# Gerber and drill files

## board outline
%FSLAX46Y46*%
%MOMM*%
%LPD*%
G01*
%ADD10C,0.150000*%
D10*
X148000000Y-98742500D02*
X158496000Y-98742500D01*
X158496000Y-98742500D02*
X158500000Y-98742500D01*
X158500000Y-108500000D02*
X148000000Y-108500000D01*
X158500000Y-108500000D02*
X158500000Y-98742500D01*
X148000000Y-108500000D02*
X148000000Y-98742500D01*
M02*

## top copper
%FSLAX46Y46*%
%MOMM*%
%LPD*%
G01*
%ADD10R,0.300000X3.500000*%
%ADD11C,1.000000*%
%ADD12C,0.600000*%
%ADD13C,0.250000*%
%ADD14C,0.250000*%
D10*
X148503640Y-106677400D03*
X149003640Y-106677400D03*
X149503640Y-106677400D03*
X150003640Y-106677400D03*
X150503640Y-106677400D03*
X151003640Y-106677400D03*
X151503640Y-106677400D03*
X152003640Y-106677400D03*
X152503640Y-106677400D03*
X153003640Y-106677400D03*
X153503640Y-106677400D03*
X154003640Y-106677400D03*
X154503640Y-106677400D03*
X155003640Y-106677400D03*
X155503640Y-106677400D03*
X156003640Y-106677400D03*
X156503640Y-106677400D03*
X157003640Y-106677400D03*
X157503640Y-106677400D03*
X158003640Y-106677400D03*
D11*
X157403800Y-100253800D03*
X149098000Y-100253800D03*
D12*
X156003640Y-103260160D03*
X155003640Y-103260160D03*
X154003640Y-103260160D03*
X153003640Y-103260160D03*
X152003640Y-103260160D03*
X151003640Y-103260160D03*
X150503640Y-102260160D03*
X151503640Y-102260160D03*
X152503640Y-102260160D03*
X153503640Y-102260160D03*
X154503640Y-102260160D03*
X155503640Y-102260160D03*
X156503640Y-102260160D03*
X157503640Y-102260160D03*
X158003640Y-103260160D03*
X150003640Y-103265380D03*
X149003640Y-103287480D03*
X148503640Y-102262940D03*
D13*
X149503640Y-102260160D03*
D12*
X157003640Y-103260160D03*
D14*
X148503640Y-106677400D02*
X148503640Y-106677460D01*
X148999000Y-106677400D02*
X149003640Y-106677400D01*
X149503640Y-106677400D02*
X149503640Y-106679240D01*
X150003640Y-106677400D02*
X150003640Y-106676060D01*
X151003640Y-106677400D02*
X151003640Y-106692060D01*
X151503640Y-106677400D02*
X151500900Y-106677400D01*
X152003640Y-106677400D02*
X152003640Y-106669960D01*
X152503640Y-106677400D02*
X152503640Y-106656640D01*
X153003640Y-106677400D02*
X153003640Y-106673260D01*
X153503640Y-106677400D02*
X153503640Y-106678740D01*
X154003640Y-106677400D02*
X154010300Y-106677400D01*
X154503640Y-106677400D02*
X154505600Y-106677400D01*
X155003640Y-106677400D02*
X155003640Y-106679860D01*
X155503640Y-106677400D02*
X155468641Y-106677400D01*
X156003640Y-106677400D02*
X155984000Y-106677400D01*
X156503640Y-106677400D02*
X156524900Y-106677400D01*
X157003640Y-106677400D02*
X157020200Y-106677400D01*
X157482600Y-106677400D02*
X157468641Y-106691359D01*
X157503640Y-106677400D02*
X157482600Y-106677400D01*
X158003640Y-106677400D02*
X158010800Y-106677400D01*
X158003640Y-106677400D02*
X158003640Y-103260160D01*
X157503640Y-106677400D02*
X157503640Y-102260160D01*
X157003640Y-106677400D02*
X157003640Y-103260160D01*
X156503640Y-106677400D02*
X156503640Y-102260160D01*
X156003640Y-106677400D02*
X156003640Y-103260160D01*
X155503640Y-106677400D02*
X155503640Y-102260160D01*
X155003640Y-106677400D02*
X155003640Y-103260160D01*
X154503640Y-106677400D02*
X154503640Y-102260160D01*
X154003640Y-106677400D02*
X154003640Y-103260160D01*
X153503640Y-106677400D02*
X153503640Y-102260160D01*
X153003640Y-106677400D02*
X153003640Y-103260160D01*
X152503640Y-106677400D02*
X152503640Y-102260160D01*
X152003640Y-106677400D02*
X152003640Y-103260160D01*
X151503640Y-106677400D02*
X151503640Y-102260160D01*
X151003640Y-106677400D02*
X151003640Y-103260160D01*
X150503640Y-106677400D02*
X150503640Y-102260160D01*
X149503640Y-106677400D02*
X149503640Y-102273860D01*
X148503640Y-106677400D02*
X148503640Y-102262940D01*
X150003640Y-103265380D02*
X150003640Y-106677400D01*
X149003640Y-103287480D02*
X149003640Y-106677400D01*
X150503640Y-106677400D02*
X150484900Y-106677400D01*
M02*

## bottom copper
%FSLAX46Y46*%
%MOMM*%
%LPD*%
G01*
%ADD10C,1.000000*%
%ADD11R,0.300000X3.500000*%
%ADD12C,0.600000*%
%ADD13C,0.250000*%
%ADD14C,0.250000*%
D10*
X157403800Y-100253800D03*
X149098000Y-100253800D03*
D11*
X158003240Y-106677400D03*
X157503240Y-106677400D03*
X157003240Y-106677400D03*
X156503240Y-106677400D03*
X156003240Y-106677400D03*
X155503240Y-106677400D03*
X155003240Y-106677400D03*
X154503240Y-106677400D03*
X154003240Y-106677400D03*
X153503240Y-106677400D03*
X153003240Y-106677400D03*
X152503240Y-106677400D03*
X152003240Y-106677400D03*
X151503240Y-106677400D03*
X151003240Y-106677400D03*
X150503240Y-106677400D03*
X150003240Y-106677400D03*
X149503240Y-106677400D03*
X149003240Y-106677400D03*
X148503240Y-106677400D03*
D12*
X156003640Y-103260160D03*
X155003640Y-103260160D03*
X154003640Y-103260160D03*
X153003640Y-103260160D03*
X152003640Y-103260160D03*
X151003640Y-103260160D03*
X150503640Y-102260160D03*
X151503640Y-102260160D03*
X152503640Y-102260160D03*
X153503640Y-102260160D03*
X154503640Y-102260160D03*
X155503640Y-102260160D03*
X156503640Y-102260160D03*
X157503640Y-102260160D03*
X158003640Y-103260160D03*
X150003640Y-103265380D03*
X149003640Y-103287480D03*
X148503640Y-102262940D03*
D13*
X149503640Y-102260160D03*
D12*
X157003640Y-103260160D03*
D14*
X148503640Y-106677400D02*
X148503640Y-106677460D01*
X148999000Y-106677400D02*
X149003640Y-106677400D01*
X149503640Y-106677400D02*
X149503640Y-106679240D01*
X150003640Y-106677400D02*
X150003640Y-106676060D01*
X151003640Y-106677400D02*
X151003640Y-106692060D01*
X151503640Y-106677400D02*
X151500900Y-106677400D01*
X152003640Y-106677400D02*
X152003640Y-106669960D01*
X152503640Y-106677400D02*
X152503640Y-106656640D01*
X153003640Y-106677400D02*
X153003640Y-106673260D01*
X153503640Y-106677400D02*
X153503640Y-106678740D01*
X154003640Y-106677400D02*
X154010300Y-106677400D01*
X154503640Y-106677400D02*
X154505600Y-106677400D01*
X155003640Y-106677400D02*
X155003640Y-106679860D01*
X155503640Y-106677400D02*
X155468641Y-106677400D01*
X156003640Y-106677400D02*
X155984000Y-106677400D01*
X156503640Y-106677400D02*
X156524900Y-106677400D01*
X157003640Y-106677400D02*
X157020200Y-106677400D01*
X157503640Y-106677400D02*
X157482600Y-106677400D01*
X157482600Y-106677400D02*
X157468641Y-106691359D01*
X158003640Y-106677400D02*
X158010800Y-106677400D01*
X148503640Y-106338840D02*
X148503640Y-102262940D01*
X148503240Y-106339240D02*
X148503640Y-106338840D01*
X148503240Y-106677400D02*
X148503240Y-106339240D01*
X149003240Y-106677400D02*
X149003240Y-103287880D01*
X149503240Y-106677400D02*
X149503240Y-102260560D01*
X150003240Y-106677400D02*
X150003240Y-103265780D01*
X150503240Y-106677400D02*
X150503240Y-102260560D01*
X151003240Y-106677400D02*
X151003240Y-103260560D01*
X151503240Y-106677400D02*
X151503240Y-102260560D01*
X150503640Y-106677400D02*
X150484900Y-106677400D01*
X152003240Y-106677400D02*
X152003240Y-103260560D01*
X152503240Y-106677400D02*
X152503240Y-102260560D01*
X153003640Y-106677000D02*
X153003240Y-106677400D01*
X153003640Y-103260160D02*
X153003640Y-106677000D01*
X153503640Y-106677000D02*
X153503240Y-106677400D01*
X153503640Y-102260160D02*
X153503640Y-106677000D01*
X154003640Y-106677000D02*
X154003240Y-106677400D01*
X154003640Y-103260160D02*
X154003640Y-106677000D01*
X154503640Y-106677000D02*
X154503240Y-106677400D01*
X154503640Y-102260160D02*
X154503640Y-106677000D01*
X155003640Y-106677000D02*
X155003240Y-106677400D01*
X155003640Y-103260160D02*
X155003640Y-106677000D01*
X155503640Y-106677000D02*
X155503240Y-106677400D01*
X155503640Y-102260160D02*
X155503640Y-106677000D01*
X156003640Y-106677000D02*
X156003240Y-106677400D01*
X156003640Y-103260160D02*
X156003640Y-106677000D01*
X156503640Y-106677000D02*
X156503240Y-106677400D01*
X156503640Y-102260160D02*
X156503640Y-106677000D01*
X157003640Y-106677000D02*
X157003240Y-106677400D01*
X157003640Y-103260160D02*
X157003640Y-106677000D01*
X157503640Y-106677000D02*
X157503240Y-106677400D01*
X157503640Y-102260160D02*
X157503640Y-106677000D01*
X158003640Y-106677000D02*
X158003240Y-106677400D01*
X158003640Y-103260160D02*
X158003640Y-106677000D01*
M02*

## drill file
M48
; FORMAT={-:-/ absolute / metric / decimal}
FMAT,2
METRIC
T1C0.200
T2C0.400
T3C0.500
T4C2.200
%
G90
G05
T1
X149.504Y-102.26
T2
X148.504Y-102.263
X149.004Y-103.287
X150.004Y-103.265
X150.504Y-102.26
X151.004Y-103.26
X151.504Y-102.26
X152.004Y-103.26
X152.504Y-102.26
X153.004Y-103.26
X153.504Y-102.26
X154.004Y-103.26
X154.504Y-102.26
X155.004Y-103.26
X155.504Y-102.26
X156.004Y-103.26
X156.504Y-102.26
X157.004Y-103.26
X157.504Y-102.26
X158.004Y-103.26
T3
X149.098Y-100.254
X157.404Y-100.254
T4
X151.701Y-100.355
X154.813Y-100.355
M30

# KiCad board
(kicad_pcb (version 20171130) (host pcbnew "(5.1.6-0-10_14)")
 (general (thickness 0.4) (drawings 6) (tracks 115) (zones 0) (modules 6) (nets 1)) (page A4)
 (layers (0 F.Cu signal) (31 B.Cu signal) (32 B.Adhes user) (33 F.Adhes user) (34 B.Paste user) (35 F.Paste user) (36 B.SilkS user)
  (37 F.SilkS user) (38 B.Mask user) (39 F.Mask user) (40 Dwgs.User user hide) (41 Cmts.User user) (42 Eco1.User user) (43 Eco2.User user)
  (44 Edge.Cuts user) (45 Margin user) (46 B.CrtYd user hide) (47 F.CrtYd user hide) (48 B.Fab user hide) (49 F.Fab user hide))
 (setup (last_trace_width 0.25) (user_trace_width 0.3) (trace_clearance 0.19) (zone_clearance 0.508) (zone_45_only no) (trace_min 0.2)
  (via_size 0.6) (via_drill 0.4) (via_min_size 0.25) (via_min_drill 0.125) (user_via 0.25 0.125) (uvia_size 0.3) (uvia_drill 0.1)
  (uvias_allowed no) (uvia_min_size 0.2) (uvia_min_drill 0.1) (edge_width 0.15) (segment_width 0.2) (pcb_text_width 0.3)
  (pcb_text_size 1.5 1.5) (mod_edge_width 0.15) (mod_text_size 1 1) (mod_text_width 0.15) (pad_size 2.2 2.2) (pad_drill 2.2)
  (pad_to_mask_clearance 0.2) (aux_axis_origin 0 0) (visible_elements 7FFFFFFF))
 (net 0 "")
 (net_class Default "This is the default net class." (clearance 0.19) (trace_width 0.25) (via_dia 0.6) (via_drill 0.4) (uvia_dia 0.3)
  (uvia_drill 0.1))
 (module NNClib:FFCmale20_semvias (layer F.Cu) (at 148.50364 104.9274)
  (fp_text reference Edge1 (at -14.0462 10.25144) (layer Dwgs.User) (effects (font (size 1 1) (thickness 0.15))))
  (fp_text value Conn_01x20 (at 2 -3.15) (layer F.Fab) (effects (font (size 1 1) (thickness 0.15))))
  (pad 1 smd rect (at 0 1.75) (size 0.3 3.5) (layers *.Paste *.Mask F.Cu))
  (pad 2 smd rect (at 0.5 1.75) (size 0.3 3.5) (layers *.Paste *.Mask F.Cu))
  (pad 3 smd rect (at 1 1.75) (size 0.3 3.5) (layers *.Paste *.Mask F.Cu))
  (pad 4 smd rect (at 1.5 1.75) (size 0.3 3.5) (layers *.Paste *.Mask F.Cu))
  (pad 5 smd rect (at 2 1.75) (size 0.3 3.5) (layers *.Paste *.Mask F.Cu))
  (pad 6 smd rect (at 2.5 1.75) (size 0.3 3.5) (layers *.Paste *.Mask F.Cu))
  (pad 7 smd rect (at 3 1.75) (size 0.3 3.5) (layers *.Paste *.Mask F.Cu))
  (pad 8 smd rect (at 3.5 1.75) (size 0.3 3.5) (layers *.Paste *.Mask F.Cu))
  (pad 9 smd rect (at 4 1.75) (size 0.3 3.5) (layers *.Paste *.Mask F.Cu))
  (pad 10 smd rect (at 4.5 1.75) (size 0.3 3.5) (layers *.Paste *.Mask F.Cu))
  (pad 11 smd rect (at 5 1.75) (size 0.3 3.5) (layers *.Paste *.Mask F.Cu))
  (pad 12 smd rect (at 5.5 1.75) (size 0.3 3.5) (layers *.Paste *.Mask F.Cu))
  (pad 13 smd rect (at 6 1.75) (size 0.3 3.5) (layers *.Paste *.Mask F.Cu))
  (pad 14 smd rect (at 6.5 1.75) (size 0.3 3.5) (layers *.Paste *.Mask F.Cu))
  (pad 15 smd rect (at 7 1.75) (size 0.3 3.5) (layers *.Paste *.Mask F.Cu))
  (pad 16 smd rect (at 7.5 1.75) (size 0.3 3.5) (layers *.Paste *.Mask F.Cu))
  (pad 17 smd rect (at 8 1.75) (size 0.3 3.5) (layers *.Paste *.Mask F.Cu))
  (pad 18 smd rect (at 8.5 1.75) (size 0.3 3.5) (layers *.Paste *.Mask F.Cu))
  (pad 19 smd rect (at 9 1.75) (size 0.3 3.5) (layers *.Paste *.Mask F.Cu))
  (pad 20 smd rect (at 9.5 1.75) (size 0.3 3.5) (layers *.Paste *.Mask F.Cu)))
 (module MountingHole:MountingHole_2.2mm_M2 (layer F.Cu) (at 151.7015 100.3554)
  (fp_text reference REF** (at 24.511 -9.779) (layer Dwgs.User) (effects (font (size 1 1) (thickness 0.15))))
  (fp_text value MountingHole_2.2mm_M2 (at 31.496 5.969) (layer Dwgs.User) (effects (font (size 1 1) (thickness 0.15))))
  (pad 1 np_thru_hole circle (at 0 0) (size 2.2 2.2) (drill 2.2) (layers *.Cu *.Mask)))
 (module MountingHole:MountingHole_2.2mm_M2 (layer F.Cu) (at 154.813 100.3554)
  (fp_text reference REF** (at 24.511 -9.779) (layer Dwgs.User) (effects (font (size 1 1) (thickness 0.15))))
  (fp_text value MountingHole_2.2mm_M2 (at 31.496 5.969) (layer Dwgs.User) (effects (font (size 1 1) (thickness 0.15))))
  (pad 1 np_thru_hole circle (at 0 0) (size 2.2 2.2) (drill 2.2) (layers *.Cu *.Mask)))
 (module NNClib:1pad (layer F.Cu) (at 157.4038 100.2538)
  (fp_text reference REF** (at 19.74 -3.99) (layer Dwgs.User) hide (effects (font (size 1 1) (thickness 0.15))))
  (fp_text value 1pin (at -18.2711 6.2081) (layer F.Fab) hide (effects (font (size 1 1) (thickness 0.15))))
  (pad 1 thru_hole circle (at 0 0) (size 1 1) (drill 0.5) (layers *.Cu *.Mask)))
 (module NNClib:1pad (layer F.Cu) (at 149.098 100.2538)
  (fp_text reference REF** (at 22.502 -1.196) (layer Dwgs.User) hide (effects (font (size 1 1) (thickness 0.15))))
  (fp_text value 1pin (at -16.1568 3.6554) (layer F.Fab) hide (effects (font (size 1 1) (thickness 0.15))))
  (pad 1 thru_hole circle (at 0 0) (size 1 1) (drill 0.5) (layers *.Cu *.Mask)))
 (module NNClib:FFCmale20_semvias (layer B.Cu) (at 158.00324 104.9274 180)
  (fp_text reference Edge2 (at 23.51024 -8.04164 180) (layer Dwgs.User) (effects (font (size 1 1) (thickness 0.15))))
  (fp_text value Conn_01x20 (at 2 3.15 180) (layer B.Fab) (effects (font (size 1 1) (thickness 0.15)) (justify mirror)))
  (pad 1 smd rect (at 0 -1.75 180) (size 0.3 3.5) (layers *.Paste *.Mask B.Cu))
  (pad 2 smd rect (at 0.5 -1.75 180) (size 0.3 3.5) (layers *.Paste *.Mask B.Cu))
  (pad 3 smd rect (at 1 -1.75 180) (size 0.3 3.5) (layers *.Paste *.Mask B.Cu))
  (pad 4 smd rect (at 1.5 -1.75 180) (size 0.3 3.5) (layers *.Paste *.Mask B.Cu))
  (pad 5 smd rect (at 2 -1.75 180) (size 0.3 3.5) (layers *.Paste *.Mask B.Cu))
  (pad 6 smd rect (at 2.5 -1.75 180) (size 0.3 3.5) (layers *.Paste *.Mask B.Cu))
  (pad 7 smd rect (at 3 -1.75 180) (size 0.3 3.5) (layers *.Paste *.Mask B.Cu))
  (pad 8 smd rect (at 3.5 -1.75 180) (size 0.3 3.5) (layers *.Paste *.Mask B.Cu))
  (pad 9 smd rect (at 4 -1.75 180) (size 0.3 3.5) (layers *.Paste *.Mask B.Cu))
  (pad 10 smd rect (at 4.5 -1.75 180) (size 0.3 3.5) (layers *.Paste *.Mask B.Cu))
  (pad 11 smd rect (at 5 -1.75 180) (size 0.3 3.5) (layers *.Paste *.Mask B.Cu))
  (pad 12 smd rect (at 5.5 -1.75 180) (size 0.3 3.5) (layers *.Paste *.Mask B.Cu))
  (pad 13 smd rect (at 6 -1.75 180) (size 0.3 3.5) (layers *.Paste *.Mask B.Cu))
  (pad 14 smd rect (at 6.5 -1.75 180) (size 0.3 3.5) (layers *.Paste *.Mask B.Cu))
  (pad 15 smd rect (at 7 -1.75 180) (size 0.3 3.5) (layers *.Paste *.Mask B.Cu))
  (pad 16 smd rect (at 7.5 -1.75 180) (size 0.3 3.5) (layers *.Paste *.Mask B.Cu))
  (pad 17 smd rect (at 8 -1.75 180) (size 0.3 3.5) (layers *.Paste *.Mask B.Cu))
  (pad 18 smd rect (at 8.5 -1.75 180) (size 0.3 3.5) (layers *.Paste *.Mask B.Cu))
  (pad 19 smd rect (at 9 -1.75 180) (size 0.3 3.5) (layers *.Paste *.Mask B.Cu))
  (pad 20 smd rect (at 9.5 -1.75 180) (size 0.3 3.5) (layers *.Paste *.Mask B.Cu)))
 (gr_line (start 148 98.7425) (end 158.496 98.7425) (layer Edge.Cuts) (width 0.15))
 (gr_line (start 158.496 98.7425) (end 158.5 98.7425) (layer Edge.Cuts) (width 0.15))
 (gr_line (start 158.5 108.5) (end 148 108.5) (angle 90) (layer Edge.Cuts) (width 0.15))
 (gr_line (start 158.5 108.5) (end 158.5 98.7425) (angle 90) (layer Edge.Cuts) (width 0.15))
 (gr_line (start 148 108.5) (end 148 98.7425) (angle 90) (layer Edge.Cuts) (width 0.15))
 (segment (start 148.50364 106.6774) (end 148.50364 106.67746) (width 0.25) (layer B.Cu) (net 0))
 (segment (start 148.999 106.6774) (end 149.00364 106.6774) (width 0.25) (layer B.Cu) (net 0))
 (segment (start 149.50364 106.6774) (end 149.50364 106.67924) (width 0.25) (layer B.Cu) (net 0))
 (segment (start 150.00364 106.6774) (end 150.00364 106.67606) (width 0.25) (layer B.Cu) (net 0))
 (segment (start 151.00364 106.6774) (end 151.00364 106.69206) (width 0.25) (layer B.Cu) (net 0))
 (segment (start 151.50364 106.6774) (end 151.5009 106.6774) (width 0.25) (layer B.Cu) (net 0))
 (segment (start 152.00364 106.6774) (end 152.00364 106.66996) (width 0.25) (layer B.Cu) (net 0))
 (segment (start 152.50364 106.6774) (end 152.50364 106.65664) (width 0.25) (layer B.Cu) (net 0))
 (segment (start 153.00364 106.6774) (end 153.00364 106.67326) (width 0.25) (layer B.Cu) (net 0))
 (segment (start 153.50364 106.6774) (end 153.50364 106.67874) (width 0.25) (layer B.Cu) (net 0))
 (segment (start 154.00364 106.6774) (end 154.0103 106.6774) (width 0.25) (layer B.Cu) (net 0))
 (segment (start 154.50364 106.6774) (end 154.5056 106.6774) (width 0.25) (layer B.Cu) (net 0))
 (segment (start 155.00364 106.6774) (end 155.00364 106.67986) (width 0.25) (layer B.Cu) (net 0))
 (segment (start 155.50364 106.6774) (end 155.468641 106.6774) (width 0.25) (layer B.Cu) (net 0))
 (segment (start 156.00364 106.6774) (end 155.984 106.6774) (width 0.25) (layer B.Cu) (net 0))
 (segment (start 156.50364 106.6774) (end 156.5249 106.6774) (width 0.25) (layer B.Cu) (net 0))
 (segment (start 157.00364 106.6774) (end 157.0202 106.6774) (width 0.25) (layer B.Cu) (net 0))
 (segment (start 157.50364 106.6774) (end 157.4826 106.6774) (width 0.25) (layer B.Cu) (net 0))
 (segment (start 157.4826 106.6774) (end 157.468641 106.691359) (width 0.25) (layer B.Cu) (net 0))
 (segment (start 158.00364 106.6774) (end 158.0108 106.6774) (width 0.25) (layer B.Cu) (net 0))
 (segment (start 148.50364 106.6774) (end 148.50364 106.67746) (width 0.25) (layer F.Cu) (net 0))
 (segment (start 148.999 106.6774) (end 149.00364 106.6774) (width 0.25) (layer F.Cu) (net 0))
 (segment (start 149.50364 106.6774) (end 149.50364 106.67924) (width 0.25) (layer F.Cu) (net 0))
 (segment (start 150.00364 106.6774) (end 150.00364 106.67606) (width 0.25) (layer F.Cu) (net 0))
 (segment (start 151.00364 106.6774) (end 151.00364 106.69206) (width 0.25) (layer F.Cu) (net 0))
 (segment (start 151.50364 106.6774) (end 151.5009 106.6774) (width 0.25) (layer F.Cu) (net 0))
 (segment (start 152.00364 106.6774) (end 152.00364 106.66996) (width 0.25) (layer F.Cu) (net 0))
 (segment (start 152.50364 106.6774) (end 152.50364 106.65664) (width 0.25) (layer F.Cu) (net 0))
 (segment (start 153.00364 106.6774) (end 153.00364 106.67326) (width 0.25) (layer F.Cu) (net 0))
 (segment (start 153.50364 106.6774) (end 153.50364 106.67874) (width 0.25) (layer F.Cu) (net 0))
 (segment (start 154.00364 106.6774) (end 154.0103 106.6774) (width 0.25) (layer F.Cu) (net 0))
 (segment (start 154.50364 106.6774) (end 154.5056 106.6774) (width 0.25) (layer F.Cu) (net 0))
 (segment (start 155.00364 106.6774) (end 155.00364 106.67986) (width 0.25) (layer F.Cu) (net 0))
 (segment (start 155.50364 106.6774) (end 155.468641 106.6774) (width 0.25) (layer F.Cu) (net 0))
 (segment (start 156.00364 106.6774) (end 155.984 106.6774) (width 0.25) (layer F.Cu) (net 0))
 (segment (start 156.50364 106.6774) (end 156.5249 106.6774) (width 0.25) (layer F.Cu) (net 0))
 (segment (start 157.00364 106.6774) (end 157.0202 106.6774) (width 0.25) (layer F.Cu) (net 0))
 (segment (start 157.4826 106.6774) (end 157.468641 106.691359) (width 0.25) (layer F.Cu) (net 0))
 (segment (start 157.50364 106.6774) (end 157.4826 106.6774) (width 0.25) (layer F.Cu) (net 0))
 (segment (start 158.00364 106.6774) (end 158.0108 106.6774) (width 0.25) (layer F.Cu) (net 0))
 (segment (start 158.00364 106.6774) (end 158.00364 103.26016) (width 0.25) (layer F.Cu) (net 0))
 (segment (start 157.50364 106.6774) (end 157.50364 102.26016) (width 0.25) (layer F.Cu) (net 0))
 (segment (start 157.00364 106.6774) (end 157.00364 103.26016) (width 0.25) (layer F.Cu) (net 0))
 (segment (start 156.50364 106.6774) (end 156.50364 102.26016) (width 0.25) (layer F.Cu) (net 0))
 (segment (start 156.00364 106.6774) (end 156.00364 103.26016) (width 0.25) (layer F.Cu) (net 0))
 (segment (start 155.50364 106.6774) (end 155.50364 102.26016) (width 0.25) (layer F.Cu) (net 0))
 (segment (start 155.00364 106.6774) (end 155.00364 103.26016) (width 0.25) (layer F.Cu) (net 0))
 (segment (start 154.50364 106.6774) (end 154.50364 102.26016) (width 0.25) (layer F.Cu) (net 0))
 (segment (start 154.00364 106.6774) (end 154.00364 103.26016) (width 0.25) (layer F.Cu) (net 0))
 (segment (start 153.50364 106.6774) (end 153.50364 102.26016) (width 0.25) (layer F.Cu) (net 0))
 (segment (start 153.00364 106.6774) (end 153.00364 103.26016) (width 0.25) (layer F.Cu) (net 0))
 (segment (start 152.50364 106.6774) (end 152.50364 102.26016) (width 0.25) (layer F.Cu) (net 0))
 (segment (start 152.00364 106.6774) (end 152.00364 103.26016) (width 0.25) (layer F.Cu) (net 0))
 (segment (start 151.50364 106.6774) (end 151.50364 102.26016) (width 0.25) (layer F.Cu) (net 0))
 (segment (start 151.00364 106.6774) (end 151.00364 103.26016) (width 0.25) (layer F.Cu) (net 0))
 (segment (start 150.50364 106.6774) (end 150.50364 102.26016) (width 0.25) (layer F.Cu) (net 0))
 (segment (start 149.50364 106.6774) (end 149.50364 102.27386) (width 0.25) (layer F.Cu) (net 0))
 (via (at 156.00364 103.26016) (size 0.6) (drill 0.4) (layers F.Cu B.Cu) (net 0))
 (via (at 155.00364 103.26016) (size 0.6) (drill 0.4) (layers F.Cu B.Cu) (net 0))
 (via (at 154.00364 103.26016) (size 0.6) (drill 0.4) (layers F.Cu B.Cu) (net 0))
 (via (at 153.00364 103.26016) (size 0.6) (drill 0.4) (layers F.Cu B.Cu) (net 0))
 (via (at 152.00364 103.26016) (size 0.6) (drill 0.4) (layers F.Cu B.Cu) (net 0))
 (via (at 151.00364 103.26016) (size 0.6) (drill 0.4) (layers F.Cu B.Cu) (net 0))
 (via (at 150.50364 102.26016) (size 0.6) (drill 0.4) (layers F.Cu B.Cu) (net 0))
 (via (at 151.50364 102.26016) (size 0.6) (drill 0.4) (layers F.Cu B.Cu) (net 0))
 (via (at 152.50364 102.26016) (size 0.6) (drill 0.4) (layers F.Cu B.Cu) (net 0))
 (via (at 153.50364 102.26016) (size 0.6) (drill 0.4) (layers F.Cu B.Cu) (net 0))
 (via (at 154.50364 102.26016) (size 0.6) (drill 0.4) (layers F.Cu B.Cu) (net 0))
 (via (at 155.50364 102.26016) (size 0.6) (drill 0.4) (layers F.Cu B.Cu) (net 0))
 (via (at 156.50364 102.26016) (size 0.6) (drill 0.4) (layers F.Cu B.Cu) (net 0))
 (via (at 157.50364 102.26016) (size 0.6) (drill 0.4) (layers F.Cu B.Cu) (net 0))
 (via (at 158.00364 103.26016) (size 0.6) (drill 0.4) (layers F.Cu B.Cu) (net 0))
 (segment (start 148.50364 106.6774) (end 148.50364 102.26294) (width 0.25) (layer F.Cu) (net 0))
 (segment (start 150.00364 103.26538) (end 150.00364 106.6774) (width 0.25) (layer F.Cu) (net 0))
 (via (at 150.00364 103.26538) (size 0.6) (drill 0.4) (layers F.Cu B.Cu) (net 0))
 (segment (start 149.00364 103.28748) (end 149.00364 106.6774) (width 0.25) (layer F.Cu) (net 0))
 (via (at 149.00364 103.28748) (size 0.6) (drill 0.4) (layers F.Cu B.Cu) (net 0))
 (via (at 148.50364 102.26294) (size 0.6) (drill 0.4) (layers F.Cu B.Cu) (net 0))
 (via (at 149.50364 102.26016) (size 0.25) (drill 0.2) (layers F.Cu B.Cu) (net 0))
 (segment (start 148.50364 106.33884) (end 148.50364 102.26294) (width 0.25) (layer B.Cu) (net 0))
 (segment (start 148.50324 106.33924) (end 148.50364 106.33884) (width 0.25) (layer B.Cu) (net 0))
 (segment (start 148.50324 106.6774) (end 148.50324 106.33924) (width 0.25) (layer B.Cu) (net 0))
 (segment (start 149.00324 106.6774) (end 149.00324 103.28788) (width 0.25) (layer B.Cu) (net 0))
 (segment (start 149.50324 106.6774) (end 149.50324 102.26056) (width 0.25) (layer B.Cu) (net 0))
 (segment (start 150.00324 106.6774) (end 150.00324 103.26578) (width 0.25) (layer B.Cu) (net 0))
 (segment (start 150.50324 106.6774) (end 150.50324 102.26056) (width 0.25) (layer B.Cu) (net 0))
 (segment (start 151.00324 106.6774) (end 151.00324 103.26056) (width 0.25) (layer B.Cu) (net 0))
 (segment (start 151.50324 106.6774) (end 151.50324 102.26056) (width 0.25) (layer B.Cu) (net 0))
 (segment (start 150.50364 106.6774) (end 150.4849 106.6774) (width 0.25) (layer F.Cu) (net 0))
 (segment (start 150.50364 106.6774) (end 150.4849 106.6774) (width 0.25) (layer B.Cu) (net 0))
 (segment (start 152.00324 106.6774) (end 152.00324 103.26056) (width 0.25) (layer B.Cu) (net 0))
 (segment (start 152.50324 106.6774) (end 152.50324 102.26056) (width 0.25) (layer B.Cu) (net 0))
 (segment (start 153.00364 106.677) (end 153.00324 106.6774) (width 0.25) (layer B.Cu) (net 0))
 (segment (start 153.00364 103.26016) (end 153.00364 106.677) (width 0.25) (layer B.Cu) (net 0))
 (segment (start 153.50364 106.677) (end 153.50324 106.6774) (width 0.25) (layer B.Cu) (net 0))
 (segment (start 153.50364 102.26016) (end 153.50364 106.677) (width 0.25) (layer B.Cu) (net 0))
 (segment (start 154.00364 106.677) (end 154.00324 106.6774) (width 0.25) (layer B.Cu) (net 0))
 (segment (start 154.00364 103.26016) (end 154.00364 106.677) (width 0.25) (layer B.Cu) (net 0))
 (segment (start 154.50364 106.677) (end 154.50324 106.6774) (width 0.25) (layer B.Cu) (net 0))
 (segment (start 154.50364 102.26016) (end 154.50364 106.677) (width 0.25) (layer B.Cu) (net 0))
 (segment (start 155.00364 106.677) (end 155.00324 106.6774) (width 0.25) (layer B.Cu) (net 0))
 (segment (start 155.00364 103.26016) (end 155.00364 106.677) (width 0.25) (layer B.Cu) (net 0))
 (segment (start 155.50364 106.677) (end 155.50324 106.6774) (width 0.25) (layer B.Cu) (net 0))
 (segment (start 155.50364 102.26016) (end 155.50364 106.677) (width 0.25) (layer B.Cu) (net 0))
 (segment (start 156.00364 106.677) (end 156.00324 106.6774) (width 0.25) (layer B.Cu) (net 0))
 (segment (start 156.00364 103.26016) (end 156.00364 106.677) (width 0.25) (layer B.Cu) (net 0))
 (segment (start 156.50364 106.677) (end 156.50324 106.6774) (width 0.25) (layer B.Cu) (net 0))
 (segment (start 156.50364 102.26016) (end 156.50364 106.677) (width 0.25) (layer B.Cu) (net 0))
 (segment (start 157.00364 106.677) (end 157.00324 106.6774) (width 0.25) (layer B.Cu) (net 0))
 (segment (start 157.00364 103.26016) (end 157.00364 106.677) (width 0.25) (layer B.Cu) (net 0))
 (segment (start 157.50364 106.677) (end 157.50324 106.6774) (width 0.25) (layer B.Cu) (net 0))
 (segment (start 157.50364 102.26016) (end 157.50364 106.677) (width 0.25) (layer B.Cu) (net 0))
 (segment (start 158.00364 106.677) (end 158.00324 106.6774) (width 0.25) (layer B.Cu) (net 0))
 (segment (start 158.00364 103.26016) (end 158.00364 106.677) (width 0.25) (layer B.Cu) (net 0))
 (via (at 157.00364 103.26016) (size 0.6) (drill 0.4) (layers F.Cu B.Cu) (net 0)))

